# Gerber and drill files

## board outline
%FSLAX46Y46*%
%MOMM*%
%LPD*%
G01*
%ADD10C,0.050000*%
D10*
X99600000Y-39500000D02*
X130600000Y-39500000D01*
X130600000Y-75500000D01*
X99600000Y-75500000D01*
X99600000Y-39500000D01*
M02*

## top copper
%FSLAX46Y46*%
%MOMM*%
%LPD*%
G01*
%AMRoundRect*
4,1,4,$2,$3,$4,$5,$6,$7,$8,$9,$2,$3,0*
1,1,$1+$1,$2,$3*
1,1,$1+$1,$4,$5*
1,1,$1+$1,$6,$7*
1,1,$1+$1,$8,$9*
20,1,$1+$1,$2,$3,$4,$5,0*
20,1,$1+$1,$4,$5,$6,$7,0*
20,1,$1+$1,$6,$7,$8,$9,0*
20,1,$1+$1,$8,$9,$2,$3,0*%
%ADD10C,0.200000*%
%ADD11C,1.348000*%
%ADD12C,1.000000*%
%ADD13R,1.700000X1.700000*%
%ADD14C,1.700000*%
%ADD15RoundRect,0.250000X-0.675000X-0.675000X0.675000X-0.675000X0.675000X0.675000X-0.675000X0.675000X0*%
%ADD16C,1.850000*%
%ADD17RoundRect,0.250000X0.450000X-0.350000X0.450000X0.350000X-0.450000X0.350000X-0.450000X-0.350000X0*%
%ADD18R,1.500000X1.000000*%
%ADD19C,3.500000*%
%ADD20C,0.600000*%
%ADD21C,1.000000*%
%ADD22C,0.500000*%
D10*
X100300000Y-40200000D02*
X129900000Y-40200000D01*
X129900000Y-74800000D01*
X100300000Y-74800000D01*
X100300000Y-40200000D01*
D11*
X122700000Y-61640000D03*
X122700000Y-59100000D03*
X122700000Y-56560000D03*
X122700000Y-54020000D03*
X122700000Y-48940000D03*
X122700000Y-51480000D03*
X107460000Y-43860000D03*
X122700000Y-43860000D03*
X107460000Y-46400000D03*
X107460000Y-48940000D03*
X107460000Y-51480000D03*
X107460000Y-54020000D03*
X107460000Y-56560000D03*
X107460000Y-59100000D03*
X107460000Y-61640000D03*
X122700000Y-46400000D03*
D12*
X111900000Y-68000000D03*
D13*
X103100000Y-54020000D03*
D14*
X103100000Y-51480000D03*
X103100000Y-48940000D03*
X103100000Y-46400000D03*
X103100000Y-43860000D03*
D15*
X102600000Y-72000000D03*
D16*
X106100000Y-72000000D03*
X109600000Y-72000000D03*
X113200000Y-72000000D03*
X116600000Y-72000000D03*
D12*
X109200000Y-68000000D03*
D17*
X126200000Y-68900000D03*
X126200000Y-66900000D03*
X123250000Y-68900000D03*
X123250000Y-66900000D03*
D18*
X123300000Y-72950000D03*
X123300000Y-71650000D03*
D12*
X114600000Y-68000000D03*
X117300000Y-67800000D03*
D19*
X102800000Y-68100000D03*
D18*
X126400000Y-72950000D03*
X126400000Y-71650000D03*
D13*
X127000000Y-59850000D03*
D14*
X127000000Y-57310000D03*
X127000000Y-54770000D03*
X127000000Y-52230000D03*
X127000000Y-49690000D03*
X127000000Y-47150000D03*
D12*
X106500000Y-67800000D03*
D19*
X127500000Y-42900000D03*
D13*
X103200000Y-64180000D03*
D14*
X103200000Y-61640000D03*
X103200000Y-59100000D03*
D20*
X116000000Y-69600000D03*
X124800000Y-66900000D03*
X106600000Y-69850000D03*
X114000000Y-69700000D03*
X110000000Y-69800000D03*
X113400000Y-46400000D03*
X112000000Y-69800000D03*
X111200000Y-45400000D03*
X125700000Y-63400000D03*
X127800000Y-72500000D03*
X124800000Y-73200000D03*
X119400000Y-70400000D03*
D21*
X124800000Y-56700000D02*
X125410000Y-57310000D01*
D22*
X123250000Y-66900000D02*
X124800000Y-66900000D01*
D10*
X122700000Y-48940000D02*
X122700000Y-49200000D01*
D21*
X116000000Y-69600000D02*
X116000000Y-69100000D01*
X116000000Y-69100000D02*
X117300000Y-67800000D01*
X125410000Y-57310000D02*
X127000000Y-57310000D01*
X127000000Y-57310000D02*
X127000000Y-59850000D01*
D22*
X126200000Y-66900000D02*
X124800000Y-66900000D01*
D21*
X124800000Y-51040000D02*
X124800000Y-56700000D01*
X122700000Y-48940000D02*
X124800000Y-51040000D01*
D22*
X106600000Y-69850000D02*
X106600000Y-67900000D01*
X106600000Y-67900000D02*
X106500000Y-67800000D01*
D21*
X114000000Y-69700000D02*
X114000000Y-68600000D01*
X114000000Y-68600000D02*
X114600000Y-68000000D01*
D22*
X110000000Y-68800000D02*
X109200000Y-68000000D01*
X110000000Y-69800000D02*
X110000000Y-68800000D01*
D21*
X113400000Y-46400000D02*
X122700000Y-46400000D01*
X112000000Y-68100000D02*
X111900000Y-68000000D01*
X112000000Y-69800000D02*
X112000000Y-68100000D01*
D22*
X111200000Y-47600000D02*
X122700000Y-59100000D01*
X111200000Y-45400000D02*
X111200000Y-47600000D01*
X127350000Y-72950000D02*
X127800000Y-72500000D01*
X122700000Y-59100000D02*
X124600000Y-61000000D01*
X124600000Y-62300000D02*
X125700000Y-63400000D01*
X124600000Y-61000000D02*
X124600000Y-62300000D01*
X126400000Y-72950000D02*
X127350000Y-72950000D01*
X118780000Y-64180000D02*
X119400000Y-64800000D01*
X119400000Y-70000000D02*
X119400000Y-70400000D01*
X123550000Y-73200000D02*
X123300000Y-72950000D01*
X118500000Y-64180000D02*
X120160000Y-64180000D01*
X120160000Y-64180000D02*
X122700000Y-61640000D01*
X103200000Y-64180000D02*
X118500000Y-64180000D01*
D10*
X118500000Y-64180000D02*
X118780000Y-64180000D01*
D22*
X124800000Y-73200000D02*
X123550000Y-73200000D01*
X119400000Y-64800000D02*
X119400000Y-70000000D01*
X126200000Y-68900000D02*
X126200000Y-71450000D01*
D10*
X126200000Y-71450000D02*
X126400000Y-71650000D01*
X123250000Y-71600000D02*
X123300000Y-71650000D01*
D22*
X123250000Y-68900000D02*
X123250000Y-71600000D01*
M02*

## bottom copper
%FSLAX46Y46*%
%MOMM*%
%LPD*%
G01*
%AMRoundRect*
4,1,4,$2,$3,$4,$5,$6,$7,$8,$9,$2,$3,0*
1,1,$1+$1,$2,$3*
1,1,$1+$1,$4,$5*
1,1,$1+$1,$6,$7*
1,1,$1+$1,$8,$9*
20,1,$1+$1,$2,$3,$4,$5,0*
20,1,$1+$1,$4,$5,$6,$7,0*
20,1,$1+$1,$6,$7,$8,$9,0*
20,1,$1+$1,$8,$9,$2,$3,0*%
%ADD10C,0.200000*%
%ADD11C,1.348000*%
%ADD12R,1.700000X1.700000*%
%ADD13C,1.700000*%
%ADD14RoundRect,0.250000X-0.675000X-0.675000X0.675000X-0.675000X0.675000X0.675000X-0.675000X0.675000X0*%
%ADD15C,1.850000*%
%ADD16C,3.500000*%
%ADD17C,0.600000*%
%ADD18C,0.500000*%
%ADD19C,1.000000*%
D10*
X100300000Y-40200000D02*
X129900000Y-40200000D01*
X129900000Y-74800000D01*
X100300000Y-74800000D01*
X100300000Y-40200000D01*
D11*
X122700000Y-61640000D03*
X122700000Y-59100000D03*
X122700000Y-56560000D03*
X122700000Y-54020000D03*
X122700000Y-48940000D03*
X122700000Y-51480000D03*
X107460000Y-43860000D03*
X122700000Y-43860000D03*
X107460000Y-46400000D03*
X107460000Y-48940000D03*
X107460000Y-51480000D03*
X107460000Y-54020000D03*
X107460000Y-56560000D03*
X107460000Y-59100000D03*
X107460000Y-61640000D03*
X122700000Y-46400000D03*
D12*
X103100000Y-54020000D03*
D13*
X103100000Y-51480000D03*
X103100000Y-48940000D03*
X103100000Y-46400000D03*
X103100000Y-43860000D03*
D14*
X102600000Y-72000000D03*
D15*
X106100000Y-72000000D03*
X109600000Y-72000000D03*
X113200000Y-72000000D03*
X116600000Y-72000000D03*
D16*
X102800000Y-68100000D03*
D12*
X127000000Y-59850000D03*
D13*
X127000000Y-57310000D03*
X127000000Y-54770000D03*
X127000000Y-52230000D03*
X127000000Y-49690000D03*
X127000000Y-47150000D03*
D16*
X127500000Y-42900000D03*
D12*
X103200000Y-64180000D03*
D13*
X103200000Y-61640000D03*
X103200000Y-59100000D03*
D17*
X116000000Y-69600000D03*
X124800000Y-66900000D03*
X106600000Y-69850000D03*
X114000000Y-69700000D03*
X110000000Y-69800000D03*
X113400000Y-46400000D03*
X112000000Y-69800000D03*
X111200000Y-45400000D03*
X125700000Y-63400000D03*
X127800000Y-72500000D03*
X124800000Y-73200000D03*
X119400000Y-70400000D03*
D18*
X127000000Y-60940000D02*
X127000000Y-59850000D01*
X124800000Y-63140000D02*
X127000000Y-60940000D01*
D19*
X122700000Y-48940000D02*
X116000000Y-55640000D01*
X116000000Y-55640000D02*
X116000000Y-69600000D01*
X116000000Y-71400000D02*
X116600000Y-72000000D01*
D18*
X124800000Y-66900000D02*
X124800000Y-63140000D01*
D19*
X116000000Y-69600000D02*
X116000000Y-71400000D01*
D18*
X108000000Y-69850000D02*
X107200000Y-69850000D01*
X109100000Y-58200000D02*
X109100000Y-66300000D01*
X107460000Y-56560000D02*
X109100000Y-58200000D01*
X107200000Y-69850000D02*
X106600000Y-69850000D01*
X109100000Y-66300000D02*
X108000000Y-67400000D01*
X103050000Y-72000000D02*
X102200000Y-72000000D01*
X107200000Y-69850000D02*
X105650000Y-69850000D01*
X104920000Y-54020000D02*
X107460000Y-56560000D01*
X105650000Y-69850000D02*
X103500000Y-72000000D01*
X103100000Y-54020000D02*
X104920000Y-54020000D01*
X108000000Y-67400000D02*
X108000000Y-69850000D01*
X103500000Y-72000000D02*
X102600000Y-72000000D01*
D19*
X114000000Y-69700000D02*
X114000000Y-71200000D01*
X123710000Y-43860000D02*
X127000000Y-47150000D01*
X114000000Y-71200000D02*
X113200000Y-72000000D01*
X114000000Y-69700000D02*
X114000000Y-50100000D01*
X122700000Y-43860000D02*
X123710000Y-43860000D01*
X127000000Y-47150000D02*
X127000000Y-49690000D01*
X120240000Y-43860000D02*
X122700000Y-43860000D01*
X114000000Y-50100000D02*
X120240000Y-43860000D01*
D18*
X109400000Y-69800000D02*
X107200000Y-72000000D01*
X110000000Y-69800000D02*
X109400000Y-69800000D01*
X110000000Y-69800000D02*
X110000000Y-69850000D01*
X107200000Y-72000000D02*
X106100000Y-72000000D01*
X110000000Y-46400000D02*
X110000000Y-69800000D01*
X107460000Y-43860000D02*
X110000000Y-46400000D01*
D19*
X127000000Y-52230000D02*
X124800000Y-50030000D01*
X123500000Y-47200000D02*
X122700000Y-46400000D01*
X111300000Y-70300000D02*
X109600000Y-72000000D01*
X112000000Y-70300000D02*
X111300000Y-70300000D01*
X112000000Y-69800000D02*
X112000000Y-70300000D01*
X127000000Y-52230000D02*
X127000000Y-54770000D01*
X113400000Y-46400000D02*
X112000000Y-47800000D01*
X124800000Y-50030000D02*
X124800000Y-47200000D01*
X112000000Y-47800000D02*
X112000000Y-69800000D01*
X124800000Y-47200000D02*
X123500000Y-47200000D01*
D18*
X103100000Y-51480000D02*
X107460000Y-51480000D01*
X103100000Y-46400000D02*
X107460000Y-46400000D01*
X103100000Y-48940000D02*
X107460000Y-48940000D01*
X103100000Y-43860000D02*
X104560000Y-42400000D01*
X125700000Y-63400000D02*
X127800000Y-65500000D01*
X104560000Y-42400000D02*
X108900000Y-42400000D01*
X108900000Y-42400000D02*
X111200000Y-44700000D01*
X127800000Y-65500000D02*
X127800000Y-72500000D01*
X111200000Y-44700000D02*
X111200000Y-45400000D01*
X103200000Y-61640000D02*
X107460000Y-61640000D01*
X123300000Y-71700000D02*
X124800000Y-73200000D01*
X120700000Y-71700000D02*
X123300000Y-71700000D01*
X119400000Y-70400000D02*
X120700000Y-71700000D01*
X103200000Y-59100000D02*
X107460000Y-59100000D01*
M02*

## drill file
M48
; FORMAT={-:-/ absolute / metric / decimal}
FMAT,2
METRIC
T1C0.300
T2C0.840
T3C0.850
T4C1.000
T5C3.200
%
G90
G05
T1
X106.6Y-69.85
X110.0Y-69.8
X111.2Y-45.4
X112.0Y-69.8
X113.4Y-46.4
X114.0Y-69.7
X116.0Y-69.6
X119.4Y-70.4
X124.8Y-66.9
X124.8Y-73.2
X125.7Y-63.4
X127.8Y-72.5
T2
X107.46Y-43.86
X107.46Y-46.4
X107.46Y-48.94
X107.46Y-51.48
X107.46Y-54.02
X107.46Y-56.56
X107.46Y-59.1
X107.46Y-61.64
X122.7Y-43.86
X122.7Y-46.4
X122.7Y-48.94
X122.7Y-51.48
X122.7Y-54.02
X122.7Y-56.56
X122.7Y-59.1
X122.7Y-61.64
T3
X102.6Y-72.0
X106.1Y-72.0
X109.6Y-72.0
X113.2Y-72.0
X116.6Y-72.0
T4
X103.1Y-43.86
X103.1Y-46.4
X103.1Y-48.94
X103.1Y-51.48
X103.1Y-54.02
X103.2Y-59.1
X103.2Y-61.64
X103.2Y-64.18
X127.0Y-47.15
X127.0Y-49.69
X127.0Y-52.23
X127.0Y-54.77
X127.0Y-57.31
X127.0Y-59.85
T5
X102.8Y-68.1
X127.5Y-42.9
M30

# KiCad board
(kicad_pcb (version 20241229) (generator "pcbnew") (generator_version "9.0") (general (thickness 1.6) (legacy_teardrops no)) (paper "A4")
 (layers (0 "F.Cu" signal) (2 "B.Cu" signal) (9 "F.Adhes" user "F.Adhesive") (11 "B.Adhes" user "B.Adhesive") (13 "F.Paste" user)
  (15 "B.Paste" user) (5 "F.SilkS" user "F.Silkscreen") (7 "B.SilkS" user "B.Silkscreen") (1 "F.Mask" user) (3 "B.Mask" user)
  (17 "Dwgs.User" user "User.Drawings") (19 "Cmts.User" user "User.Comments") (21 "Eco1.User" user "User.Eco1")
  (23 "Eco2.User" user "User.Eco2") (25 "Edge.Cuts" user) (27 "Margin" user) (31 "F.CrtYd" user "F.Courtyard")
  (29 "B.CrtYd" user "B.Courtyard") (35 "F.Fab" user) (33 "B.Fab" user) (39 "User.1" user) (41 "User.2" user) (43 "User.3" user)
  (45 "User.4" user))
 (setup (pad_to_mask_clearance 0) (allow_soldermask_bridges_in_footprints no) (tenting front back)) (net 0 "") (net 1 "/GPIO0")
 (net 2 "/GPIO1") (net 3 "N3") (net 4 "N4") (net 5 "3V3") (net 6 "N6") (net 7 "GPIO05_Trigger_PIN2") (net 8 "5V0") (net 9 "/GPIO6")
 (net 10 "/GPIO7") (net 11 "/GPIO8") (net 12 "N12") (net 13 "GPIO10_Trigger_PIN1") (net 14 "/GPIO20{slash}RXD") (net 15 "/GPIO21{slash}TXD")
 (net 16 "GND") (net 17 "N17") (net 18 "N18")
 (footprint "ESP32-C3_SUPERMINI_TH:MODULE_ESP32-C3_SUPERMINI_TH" (layer "F.Cu") (at 115.08 53.76)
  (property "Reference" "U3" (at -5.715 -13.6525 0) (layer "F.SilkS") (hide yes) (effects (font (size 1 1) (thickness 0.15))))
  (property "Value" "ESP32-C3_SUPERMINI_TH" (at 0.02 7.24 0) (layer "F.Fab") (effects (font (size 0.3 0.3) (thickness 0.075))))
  (pad "0" thru_hole circle (at 7.62 7.88) (size 1.348 1.348) (drill 0.84) (layers "*.Cu" "*.Mask") (remove_unused_layers no)
   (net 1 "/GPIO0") (solder_mask_margin 0.102))
  (pad "1" thru_hole circle (at 7.62 5.34) (size 1.348 1.348) (drill 0.84) (layers "*.Cu" "*.Mask") (remove_unused_layers no)
   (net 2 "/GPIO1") (solder_mask_margin 0.102))
  (pad "2" thru_hole circle (at 7.62 2.8) (size 1.348 1.348) (drill 0.84) (layers "*.Cu" "*.Mask") (remove_unused_layers no) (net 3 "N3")
   (solder_mask_margin 0.102))
  (pad "3" thru_hole circle (at 7.62 0.26) (size 1.348 1.348) (drill 0.84) (layers "*.Cu" "*.Mask") (remove_unused_layers no) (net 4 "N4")
   (solder_mask_margin 0.102))
  (pad "3.3" thru_hole circle (at 7.62 -4.82) (size 1.348 1.348) (drill 0.84) (layers "*.Cu" "*.Mask") (remove_unused_layers no)
   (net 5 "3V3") (solder_mask_margin 0.102))
  (pad "4" thru_hole circle (at 7.62 -2.28) (size 1.348 1.348) (drill 0.84) (layers "*.Cu" "*.Mask") (remove_unused_layers no) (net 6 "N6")
   (solder_mask_margin 0.102))
  (pad "5" thru_hole circle (at -7.62 -9.9) (size 1.348 1.348) (drill 0.84) (layers "*.Cu" "*.Mask") (remove_unused_layers no)
   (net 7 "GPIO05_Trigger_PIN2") (solder_mask_margin 0.102))
  (pad "5V" thru_hole circle (at 7.62 -9.9) (size 1.348 1.348) (drill 0.84) (layers "*.Cu" "*.Mask") (remove_unused_layers no) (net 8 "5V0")
   (solder_mask_margin 0.102))
  (pad "6" thru_hole circle (at -7.62 -7.36) (size 1.348 1.348) (drill 0.84) (layers "*.Cu" "*.Mask") (remove_unused_layers no)
   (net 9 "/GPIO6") (solder_mask_margin 0.102))
  (pad "7" thru_hole circle (at -7.62 -4.82) (size 1.348 1.348) (drill 0.84) (layers "*.Cu" "*.Mask") (remove_unused_layers no)
   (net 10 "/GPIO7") (solder_mask_margin 0.102))
  (pad "8" thru_hole circle (at -7.62 -2.28) (size 1.348 1.348) (drill 0.84) (layers "*.Cu" "*.Mask") (remove_unused_layers no)
   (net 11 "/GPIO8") (solder_mask_margin 0.102))
  (pad "9" thru_hole circle (at -7.62 0.26) (size 1.348 1.348) (drill 0.84) (layers "*.Cu" "*.Mask") (remove_unused_layers no)
   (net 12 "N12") (solder_mask_margin 0.102))
  (pad "10" thru_hole circle (at -7.62 2.8) (size 1.348 1.348) (drill 0.84) (layers "*.Cu" "*.Mask") (remove_unused_layers no)
   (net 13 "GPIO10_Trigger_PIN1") (solder_mask_margin 0.102))
  (pad "20" thru_hole circle (at -7.62 5.34) (size 1.348 1.348) (drill 0.84) (layers "*.Cu" "*.Mask") (remove_unused_layers no)
   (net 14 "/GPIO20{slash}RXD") (solder_mask_margin 0.102))
  (pad "21" thru_hole circle (at -7.62 7.88) (size 1.348 1.348) (drill 0.84) (layers "*.Cu" "*.Mask") (remove_unused_layers no)
   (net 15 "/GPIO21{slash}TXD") (solder_mask_margin 0.102))
  (pad "G" thru_hole circle (at 7.62 -7.36) (size 1.348 1.348) (drill 0.84) (layers "*.Cu" "*.Mask") (remove_unused_layers no)
   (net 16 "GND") (solder_mask_margin 0.102)))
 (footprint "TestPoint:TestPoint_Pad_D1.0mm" (layer "F.Cu") (at 111.9 68)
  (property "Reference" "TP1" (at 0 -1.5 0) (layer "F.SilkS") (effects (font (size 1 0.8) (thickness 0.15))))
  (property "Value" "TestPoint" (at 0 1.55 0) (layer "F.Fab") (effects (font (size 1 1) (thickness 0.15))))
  (pad "1" smd circle (at 0 0) (size 1 1) (layers "F.Cu" "F.Mask") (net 16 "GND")))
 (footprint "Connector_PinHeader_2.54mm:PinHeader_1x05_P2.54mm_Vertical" (layer "F.Cu") (at 103.1 54.02 180)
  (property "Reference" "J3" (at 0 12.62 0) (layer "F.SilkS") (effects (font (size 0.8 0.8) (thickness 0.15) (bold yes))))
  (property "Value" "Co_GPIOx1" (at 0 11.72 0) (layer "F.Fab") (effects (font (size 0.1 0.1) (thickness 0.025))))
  (pad "1" thru_hole rect (at 0 0 180) (size 1.7 1.7) (drill 1) (layers "*.Cu" "*.Mask") (remove_unused_layers no)
   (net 13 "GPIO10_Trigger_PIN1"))
  (pad "2" thru_hole circle (at 0 2.54 180) (size 1.7 1.7) (drill 1) (layers "*.Cu" "*.Mask") (remove_unused_layers no) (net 11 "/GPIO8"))
  (pad "3" thru_hole circle (at 0 5.08 180) (size 1.7 1.7) (drill 1) (layers "*.Cu" "*.Mask") (remove_unused_layers no) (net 10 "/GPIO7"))
  (pad "4" thru_hole circle (at 0 7.62 180) (size 1.7 1.7) (drill 1) (layers "*.Cu" "*.Mask") (remove_unused_layers no) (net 9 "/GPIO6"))
  (pad "5" thru_hole circle (at 0 10.16 180) (size 1.7 1.7) (drill 1) (layers "*.Cu" "*.Mask") (remove_unused_layers no) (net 2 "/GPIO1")))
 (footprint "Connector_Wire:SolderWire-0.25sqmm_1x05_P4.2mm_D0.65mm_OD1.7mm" (layer "F.Cu") (at 109.6 72)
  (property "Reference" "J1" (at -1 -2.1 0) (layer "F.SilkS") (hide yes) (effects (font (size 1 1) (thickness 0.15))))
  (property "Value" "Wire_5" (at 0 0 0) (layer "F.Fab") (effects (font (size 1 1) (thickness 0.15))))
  (pad "1" thru_hole roundrect (at -7 0) (size 1.85 1.85) (drill 0.85) (layers "*.Cu" "*.Mask") (remove_unused_layers no)
   (roundrect_rratio 0.135135) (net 13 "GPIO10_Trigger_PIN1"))
  (pad "2" thru_hole circle (at -3.5 0) (size 1.85 1.85) (drill 0.85) (layers "*.Cu" "*.Mask") (remove_unused_layers no)
   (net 7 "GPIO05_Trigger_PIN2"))
  (pad "3" thru_hole circle (at 0 0) (size 1.85 1.85) (drill 0.85) (layers "*.Cu" "*.Mask") (remove_unused_layers no) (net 16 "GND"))
  (pad "4" thru_hole circle (at 3.6 0) (size 1.85 1.85) (drill 0.85) (layers "*.Cu" "*.Mask") (remove_unused_layers no) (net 8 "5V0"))
  (pad "5" thru_hole circle (at 7 0) (size 1.85 1.85) (drill 0.85) (layers "*.Cu" "*.Mask") (remove_unused_layers no) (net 5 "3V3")))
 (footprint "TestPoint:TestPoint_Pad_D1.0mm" (layer "F.Cu") (at 109.2 68)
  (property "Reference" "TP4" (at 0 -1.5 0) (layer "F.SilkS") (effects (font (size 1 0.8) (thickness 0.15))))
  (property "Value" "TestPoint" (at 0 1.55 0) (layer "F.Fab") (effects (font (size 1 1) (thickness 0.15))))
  (pad "1" smd circle (at 0 0) (size 1 1) (layers "F.Cu" "F.Mask") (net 7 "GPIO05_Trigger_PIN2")))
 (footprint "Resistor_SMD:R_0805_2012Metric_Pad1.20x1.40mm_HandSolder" (layer "F.Cu") (at 126.2 67.9 90)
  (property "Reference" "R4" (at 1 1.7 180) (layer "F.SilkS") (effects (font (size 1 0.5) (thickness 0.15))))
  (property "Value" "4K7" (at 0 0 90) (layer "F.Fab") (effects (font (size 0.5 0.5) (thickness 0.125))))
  (pad "1" smd roundrect (at -1 0 90) (size 1.2 1.4) (layers "F.Cu" "F.Mask" "F.Paste") (roundrect_rratio 0.208333) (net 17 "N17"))
  (pad "2" smd roundrect (at 1 0 90) (size 1.2 1.4) (layers "F.Cu" "F.Mask" "F.Paste") (roundrect_rratio 0.208333) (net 5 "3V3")))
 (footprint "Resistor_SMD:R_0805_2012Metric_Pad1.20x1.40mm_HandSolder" (layer "F.Cu") (at 123.25 67.9 90)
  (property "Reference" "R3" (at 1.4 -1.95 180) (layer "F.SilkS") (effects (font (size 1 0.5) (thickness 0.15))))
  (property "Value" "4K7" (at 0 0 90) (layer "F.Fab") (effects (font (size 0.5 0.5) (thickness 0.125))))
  (pad "1" smd roundrect (at -1 0 90) (size 1.2 1.4) (layers "F.Cu" "F.Mask" "F.Paste") (roundrect_rratio 0.208333) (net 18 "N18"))
  (pad "2" smd roundrect (at 1 0 90) (size 1.2 1.4) (layers "F.Cu" "F.Mask" "F.Paste") (roundrect_rratio 0.208333) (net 5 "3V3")))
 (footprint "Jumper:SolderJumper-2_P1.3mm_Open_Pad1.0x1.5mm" (layer "F.Cu") (at 123.3 72.3 90)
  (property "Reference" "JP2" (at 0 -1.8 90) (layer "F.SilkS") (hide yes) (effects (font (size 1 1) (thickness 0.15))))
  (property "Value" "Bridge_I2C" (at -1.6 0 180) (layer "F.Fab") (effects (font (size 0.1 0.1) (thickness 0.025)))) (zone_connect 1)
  (pad "1" smd rect (at -0.65 0 90) (size 1 1.5) (layers "F.Cu" "F.Mask") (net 1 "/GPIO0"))
  (pad "2" smd rect (at 0.65 0 90) (size 1 1.5) (layers "F.Cu" "F.Mask") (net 18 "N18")))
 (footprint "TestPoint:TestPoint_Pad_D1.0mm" (layer "F.Cu") (at 114.6 68)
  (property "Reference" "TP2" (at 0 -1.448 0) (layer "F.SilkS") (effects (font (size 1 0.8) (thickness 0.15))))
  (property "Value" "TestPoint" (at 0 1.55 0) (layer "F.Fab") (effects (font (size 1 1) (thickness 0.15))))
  (pad "1" smd circle (at 0 0) (size 1 1) (layers "F.Cu" "F.Mask") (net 8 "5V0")))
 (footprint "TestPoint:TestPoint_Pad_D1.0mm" (layer "F.Cu") (at 117.3 67.8)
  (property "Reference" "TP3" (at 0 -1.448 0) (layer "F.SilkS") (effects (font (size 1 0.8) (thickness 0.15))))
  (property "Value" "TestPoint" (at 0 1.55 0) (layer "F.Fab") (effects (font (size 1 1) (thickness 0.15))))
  (pad "1" smd circle (at 0 0) (size 1 1) (layers "F.Cu" "F.Mask") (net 5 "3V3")))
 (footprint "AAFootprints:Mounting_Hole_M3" (layer "F.Cu") (at 102.8 68.1)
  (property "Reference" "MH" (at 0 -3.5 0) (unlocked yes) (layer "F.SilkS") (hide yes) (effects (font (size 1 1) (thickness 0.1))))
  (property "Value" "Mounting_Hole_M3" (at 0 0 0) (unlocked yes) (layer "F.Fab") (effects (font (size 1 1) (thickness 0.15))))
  (pad "" np_thru_hole circle (at 0 0) (size 3.5 3.5) (drill 3.2) (layers "*.Cu" "*.Mask")))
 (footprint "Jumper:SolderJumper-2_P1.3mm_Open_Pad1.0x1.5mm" (layer "F.Cu") (at 126.4 72.3 90)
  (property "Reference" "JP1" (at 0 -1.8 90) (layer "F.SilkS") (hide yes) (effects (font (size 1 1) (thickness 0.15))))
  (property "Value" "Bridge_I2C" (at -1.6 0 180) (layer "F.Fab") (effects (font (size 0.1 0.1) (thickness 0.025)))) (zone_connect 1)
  (pad "1" smd rect (at -0.65 0 90) (size 1 1.5) (layers "F.Cu" "F.Mask") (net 2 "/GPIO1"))
  (pad "2" smd rect (at 0.65 0 90) (size 1 1.5) (layers "F.Cu" "F.Mask") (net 17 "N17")))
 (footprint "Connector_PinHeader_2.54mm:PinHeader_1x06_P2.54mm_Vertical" (layer "F.Cu") (at 127 59.85 180)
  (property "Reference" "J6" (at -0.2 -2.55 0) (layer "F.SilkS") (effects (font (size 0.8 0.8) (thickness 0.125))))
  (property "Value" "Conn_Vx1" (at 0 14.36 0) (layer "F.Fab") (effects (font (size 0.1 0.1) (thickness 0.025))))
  (pad "1" thru_hole rect (at 0 0 180) (size 1.7 1.7) (drill 1) (layers "*.Cu" "*.Mask") (remove_unused_layers no) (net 5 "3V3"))
  (pad "2" thru_hole circle (at 0 2.54 180) (size 1.7 1.7) (drill 1) (layers "*.Cu" "*.Mask") (remove_unused_layers no) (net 5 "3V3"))
  (pad "3" thru_hole circle (at 0 5.08 180) (size 1.7 1.7) (drill 1) (layers "*.Cu" "*.Mask") (remove_unused_layers no) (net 16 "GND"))
  (pad "4" thru_hole circle (at 0 7.62 180) (size 1.7 1.7) (drill 1) (layers "*.Cu" "*.Mask") (remove_unused_layers no) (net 16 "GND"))
  (pad "5" thru_hole circle (at 0 10.16 180) (size 1.7 1.7) (drill 1) (layers "*.Cu" "*.Mask") (remove_unused_layers no) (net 8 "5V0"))
  (pad "6" thru_hole circle (at 0 12.7 180) (size 1.7 1.7) (drill 1) (layers "*.Cu" "*.Mask") (remove_unused_layers no) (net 8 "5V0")))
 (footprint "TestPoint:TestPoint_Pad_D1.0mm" (layer "F.Cu") (at 106.5 67.8)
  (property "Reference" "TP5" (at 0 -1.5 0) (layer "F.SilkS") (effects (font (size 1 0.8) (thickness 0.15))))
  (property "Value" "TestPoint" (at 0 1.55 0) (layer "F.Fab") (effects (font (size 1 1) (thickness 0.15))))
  (pad "1" smd circle (at 0 0) (size 1 1) (layers "F.Cu" "F.Mask") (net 13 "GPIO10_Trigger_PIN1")))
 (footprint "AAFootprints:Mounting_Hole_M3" (layer "F.Cu") (at 127.5 42.9)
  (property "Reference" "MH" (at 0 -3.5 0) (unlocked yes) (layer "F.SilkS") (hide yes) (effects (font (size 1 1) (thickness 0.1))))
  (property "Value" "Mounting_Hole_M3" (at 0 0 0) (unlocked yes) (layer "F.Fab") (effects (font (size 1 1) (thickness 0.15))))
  (pad "" np_thru_hole circle (at 0 0) (size 3.5 3.5) (drill 3.2) (layers "*.Cu" "*.Mask")))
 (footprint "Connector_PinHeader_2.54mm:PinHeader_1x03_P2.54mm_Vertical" (layer "F.Cu") (at 103.2 64.18 180)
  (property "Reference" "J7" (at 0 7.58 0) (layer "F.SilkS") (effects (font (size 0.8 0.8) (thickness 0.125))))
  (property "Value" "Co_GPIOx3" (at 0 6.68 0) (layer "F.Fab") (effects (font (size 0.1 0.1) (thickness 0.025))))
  (pad "1" thru_hole rect (at 0 0 180) (size 1.7 1.7) (drill 1) (layers "*.Cu" "*.Mask") (remove_unused_layers no) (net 1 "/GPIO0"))
  (pad "2" thru_hole circle (at 0 2.54 180) (size 1.7 1.7) (drill 1) (layers "*.Cu" "*.Mask") (remove_unused_layers no)
   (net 15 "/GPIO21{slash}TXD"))
  (pad "3" thru_hole circle (at 0 5.08 180) (size 1.7 1.7) (drill 1) (layers "*.Cu" "*.Mask") (remove_unused_layers no)
   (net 14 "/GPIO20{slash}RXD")))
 (gr_rect (start 100.3 40.2) (end 129.9 74.8) (stroke (width 0.2) (type solid)) (fill no) (layer "F.Cu") (net 16))
 (gr_rect (start 100.3 40.2) (end 129.9 74.8) (stroke (width 0.2) (type default)) (fill no) (layer "B.Cu") (net 16))
 (gr_rect (start 99.6 39.5) (end 130.6 75.5) (stroke (width 0.05) (type solid)) (fill no) (layer "Edge.Cuts"))
 (segment (start 124.8 56.7) (end 125.41 57.31) (width 1) (layer "F.Cu") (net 5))
 (segment (start 123.25 66.9) (end 124.8 66.9) (width 0.5) (layer "F.Cu") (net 5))
 (segment (start 122.7 48.94) (end 122.7 49.2) (width 0.2) (layer "F.Cu") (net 5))
 (segment (start 116 69.6) (end 116 69.1) (width 1) (layer "F.Cu") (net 5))
 (segment (start 116 69.1) (end 117.3 67.8) (width 1) (layer "F.Cu") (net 5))
 (segment (start 125.41 57.31) (end 127 57.31) (width 1) (layer "F.Cu") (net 5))
 (segment (start 127 57.31) (end 127 59.85) (width 1) (layer "F.Cu") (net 5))
 (segment (start 126.2 66.9) (end 124.8 66.9) (width 0.5) (layer "F.Cu") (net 5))
 (segment (start 124.8 51.04) (end 124.8 56.7) (width 1) (layer "F.Cu") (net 5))
 (segment (start 122.7 48.94) (end 124.8 51.04) (width 1) (layer "F.Cu") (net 5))
 (via (at 116 69.6) (size 0.6) (drill 0.3) (layers "F.Cu" "B.Cu") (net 5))
 (via (at 124.8 66.9) (size 0.6) (drill 0.3) (layers "F.Cu" "B.Cu") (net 5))
 (segment (start 127 60.94) (end 127 59.85) (width 0.5) (layer "B.Cu") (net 5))
 (segment (start 124.8 63.14) (end 127 60.94) (width 0.5) (layer "B.Cu") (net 5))
 (segment (start 122.7 48.94) (end 116 55.64) (width 1) (layer "B.Cu") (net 5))
 (segment (start 116 55.64) (end 116 69.6) (width 1) (layer "B.Cu") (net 5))
 (segment (start 116 71.4) (end 116.6 72) (width 1) (layer "B.Cu") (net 5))
 (segment (start 124.8 66.9) (end 124.8 63.14) (width 0.5) (layer "B.Cu") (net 5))
 (segment (start 116 69.6) (end 116 71.4) (width 1) (layer "B.Cu") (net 5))
 (segment (start 106.6 69.85) (end 106.6 67.9) (width 0.5) (layer "F.Cu") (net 13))
 (segment (start 106.6 67.9) (end 106.5 67.8) (width 0.5) (layer "F.Cu") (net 13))
 (via (at 106.6 69.85) (size 0.6) (drill 0.3) (layers "F.Cu" "B.Cu") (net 13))
 (segment (start 108 69.85) (end 107.2 69.85) (width 0.5) (layer "B.Cu") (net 13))
 (segment (start 109.1 58.2) (end 109.1 66.3) (width 0.5) (layer "B.Cu") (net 13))
 (segment (start 107.46 56.56) (end 109.1 58.2) (width 0.5) (layer "B.Cu") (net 13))
 (segment (start 107.2 69.85) (end 106.6 69.85) (width 0.5) (layer "B.Cu") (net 13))
 (segment (start 109.1 66.3) (end 108 67.4) (width 0.5) (layer "B.Cu") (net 13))
 (segment (start 103.05 72) (end 102.2 72) (width 0.5) (layer "B.Cu") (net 13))
 (segment (start 107.2 69.85) (end 105.65 69.85) (width 0.5) (layer "B.Cu") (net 13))
 (segment (start 104.92 54.02) (end 107.46 56.56) (width 0.5) (layer "B.Cu") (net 13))
 (segment (start 105.65 69.85) (end 103.5 72) (width 0.5) (layer "B.Cu") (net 13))
 (segment (start 103.1 54.02) (end 104.92 54.02) (width 0.5) (layer "B.Cu") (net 13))
 (segment (start 108 67.4) (end 108 69.85) (width 0.5) (layer "B.Cu") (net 13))
 (segment (start 103.5 72) (end 102.6 72) (width 0.5) (layer "B.Cu") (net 13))
 (segment (start 114 69.7) (end 114 68.6) (width 1) (layer "F.Cu") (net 8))
 (segment (start 114 68.6) (end 114.6 68) (width 1) (layer "F.Cu") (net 8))
 (via (at 114 69.7) (size 0.6) (drill 0.3) (layers "F.Cu" "B.Cu") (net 8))
 (segment (start 114 69.7) (end 114 71.2) (width 1) (layer "B.Cu") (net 8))
 (segment (start 123.71 43.86) (end 127 47.15) (width 1) (layer "B.Cu") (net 8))
 (segment (start 114 71.2) (end 113.2 72) (width 1) (layer "B.Cu") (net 8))
 (segment (start 114 69.7) (end 114 50.1) (width 1) (layer "B.Cu") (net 8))
 (segment (start 122.7 43.86) (end 123.71 43.86) (width 1) (layer "B.Cu") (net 8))
 (segment (start 127 47.15) (end 127 49.69) (width 1) (layer "B.Cu") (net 8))
 (segment (start 120.24 43.86) (end 122.7 43.86) (width 1) (layer "B.Cu") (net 8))
 (segment (start 114 50.1) (end 120.24 43.86) (width 1) (layer "B.Cu") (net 8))
 (segment (start 110 68.8) (end 109.2 68) (width 0.5) (layer "F.Cu") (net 7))
 (segment (start 110 69.8) (end 110 68.8) (width 0.5) (layer "F.Cu") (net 7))
 (via (at 110 69.8) (size 0.6) (drill 0.3) (layers "F.Cu" "B.Cu") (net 7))
 (segment (start 109.4 69.8) (end 107.2 72) (width 0.5) (layer "B.Cu") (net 7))
 (segment (start 110 69.8) (end 109.4 69.8) (width 0.5) (layer "B.Cu") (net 7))
 (segment (start 110 69.8) (end 110 69.85) (width 0.5) (layer "B.Cu") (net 7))
 (segment (start 107.2 72) (end 106.1 72) (width 0.5) (layer "B.Cu") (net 7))
 (segment (start 110 46.4) (end 110 69.8) (width 0.5) (layer "B.Cu") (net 7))
 (segment (start 107.46 43.86) (end 110 46.4) (width 0.5) (layer "B.Cu") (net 7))
 (segment (start 113.4 46.4) (end 122.7 46.4) (width 1) (layer "F.Cu") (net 16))
 (segment (start 112 68.1) (end 111.9 68) (width 1) (layer "F.Cu") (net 16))
 (segment (start 112 69.8) (end 112 68.1) (width 1) (layer "F.Cu") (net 16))
 (via (at 113.4 46.4) (size 0.6) (drill 0.3) (layers "F.Cu" "B.Cu") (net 16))
 (via (at 112 69.8) (size 0.6) (drill 0.3) (layers "F.Cu" "B.Cu") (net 16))
 (segment (start 127 52.23) (end 124.8 50.03) (width 1) (layer "B.Cu") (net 16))
 (segment (start 123.5 47.2) (end 122.7 46.4) (width 1) (layer "B.Cu") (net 16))
 (segment (start 111.3 70.3) (end 109.6 72) (width 1) (layer "B.Cu") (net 16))
 (segment (start 112 70.3) (end 111.3 70.3) (width 1) (layer "B.Cu") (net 16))
 (segment (start 112 69.8) (end 112 70.3) (width 1) (layer "B.Cu") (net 16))
 (segment (start 127 52.23) (end 127 54.77) (width 1) (layer "B.Cu") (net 16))
 (segment (start 113.4 46.4) (end 112 47.8) (width 1) (layer "B.Cu") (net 16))
 (segment (start 124.8 50.03) (end 124.8 47.2) (width 1) (layer "B.Cu") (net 16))
 (segment (start 112 47.8) (end 112 69.8) (width 1) (layer "B.Cu") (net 16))
 (segment (start 124.8 47.2) (end 123.5 47.2) (width 1) (layer "B.Cu") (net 16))
 (segment (start 103.1 51.48) (end 107.46 51.48) (width 0.5) (layer "B.Cu") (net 11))
 (segment (start 103.1 46.4) (end 107.46 46.4) (width 0.5) (layer "B.Cu") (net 9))
 (segment (start 103.1 48.94) (end 107.46 48.94) (width 0.5) (layer "B.Cu") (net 10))
 (segment (start 111.2 47.6) (end 122.7 59.1) (width 0.5) (layer "F.Cu") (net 2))
 (segment (start 111.2 45.4) (end 111.2 47.6) (width 0.5) (layer "F.Cu") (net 2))
 (segment (start 127.35 72.95) (end 127.8 72.5) (width 0.5) (layer "F.Cu") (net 2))
 (segment (start 122.7 59.1) (end 124.6 61) (width 0.5) (layer "F.Cu") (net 2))
 (segment (start 124.6 62.3) (end 125.7 63.4) (width 0.5) (layer "F.Cu") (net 2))
 (segment (start 124.6 61) (end 124.6 62.3) (width 0.5) (layer "F.Cu") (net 2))
 (segment (start 126.4 72.95) (end 127.35 72.95) (width 0.5) (layer "F.Cu") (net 2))
 (via (at 111.2 45.4) (size 0.6) (drill 0.3) (layers "F.Cu" "B.Cu") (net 2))
 (via (at 125.7 63.4) (size 0.6) (drill 0.3) (layers "F.Cu" "B.Cu") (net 2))
 (via (at 127.8 72.5) (size 0.6) (drill 0.3) (layers "F.Cu" "B.Cu") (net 2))
 (segment (start 103.1 43.86) (end 104.56 42.4) (width 0.5) (layer "B.Cu") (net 2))
 (segment (start 125.7 63.4) (end 127.8 65.5) (width 0.5) (layer "B.Cu") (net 2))
 (segment (start 104.56 42.4) (end 108.9 42.4) (width 0.5) (layer "B.Cu") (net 2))
 (segment (start 108.9 42.4) (end 111.2 44.7) (width 0.5) (layer "B.Cu") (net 2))
 (segment (start 127.8 65.5) (end 127.8 72.5) (width 0.5) (layer "B.Cu") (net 2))
 (segment (start 111.2 44.7) (end 111.2 45.4) (width 0.5) (layer "B.Cu") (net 2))
 (segment (start 103.2 61.64) (end 107.46 61.64) (width 0.5) (layer "B.Cu") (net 15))
 (segment (start 118.78 64.18) (end 119.4 64.8) (width 0.5) (layer "F.Cu") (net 1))
 (segment (start 119.4 70) (end 119.4 70.4) (width 0.5) (layer "F.Cu") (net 1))
 (segment (start 123.55 73.2) (end 123.3 72.95) (width 0.5) (layer "F.Cu") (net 1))
 (segment (start 118.5 64.18) (end 120.16 64.18) (width 0.5) (layer "F.Cu") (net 1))
 (segment (start 120.16 64.18) (end 122.7 61.64) (width 0.5) (layer "F.Cu") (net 1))
 (segment (start 103.2 64.18) (end 118.5 64.18) (width 0.5) (layer "F.Cu") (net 1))
 (segment (start 118.5 64.18) (end 118.78 64.18) (width 0.2) (layer "F.Cu") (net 1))
 (segment (start 124.8 73.2) (end 123.55 73.2) (width 0.5) (layer "F.Cu") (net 1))
 (segment (start 119.4 64.8) (end 119.4 70) (width 0.5) (layer "F.Cu") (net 1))
 (via (at 124.8 73.2) (size 0.6) (drill 0.3) (layers "F.Cu" "B.Cu") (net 1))
 (via (at 119.4 70.4) (size 0.6) (drill 0.3) (layers "F.Cu" "B.Cu") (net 1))
 (segment (start 123.3 71.7) (end 124.8 73.2) (width 0.5) (layer "B.Cu") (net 1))
 (segment (start 120.7 71.7) (end 123.3 71.7) (width 0.5) (layer "B.Cu") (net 1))
 (segment (start 119.4 70.4) (end 120.7 71.7) (width 0.5) (layer "B.Cu") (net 1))
 (segment (start 103.2 59.1) (end 107.46 59.1) (width 0.5) (layer "B.Cu") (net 14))
 (segment (start 126.2 68.9) (end 126.2 71.45) (width 0.5) (layer "F.Cu") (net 17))
 (segment (start 126.2 71.45) (end 126.4 71.65) (width 0.2) (layer "F.Cu") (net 17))
 (segment (start 123.25 71.6) (end 123.3 71.65) (width 0.2) (layer "F.Cu") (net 18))
 (segment (start 123.25 68.9) (end 123.25 71.6) (width 0.5) (layer "F.Cu") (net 18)))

